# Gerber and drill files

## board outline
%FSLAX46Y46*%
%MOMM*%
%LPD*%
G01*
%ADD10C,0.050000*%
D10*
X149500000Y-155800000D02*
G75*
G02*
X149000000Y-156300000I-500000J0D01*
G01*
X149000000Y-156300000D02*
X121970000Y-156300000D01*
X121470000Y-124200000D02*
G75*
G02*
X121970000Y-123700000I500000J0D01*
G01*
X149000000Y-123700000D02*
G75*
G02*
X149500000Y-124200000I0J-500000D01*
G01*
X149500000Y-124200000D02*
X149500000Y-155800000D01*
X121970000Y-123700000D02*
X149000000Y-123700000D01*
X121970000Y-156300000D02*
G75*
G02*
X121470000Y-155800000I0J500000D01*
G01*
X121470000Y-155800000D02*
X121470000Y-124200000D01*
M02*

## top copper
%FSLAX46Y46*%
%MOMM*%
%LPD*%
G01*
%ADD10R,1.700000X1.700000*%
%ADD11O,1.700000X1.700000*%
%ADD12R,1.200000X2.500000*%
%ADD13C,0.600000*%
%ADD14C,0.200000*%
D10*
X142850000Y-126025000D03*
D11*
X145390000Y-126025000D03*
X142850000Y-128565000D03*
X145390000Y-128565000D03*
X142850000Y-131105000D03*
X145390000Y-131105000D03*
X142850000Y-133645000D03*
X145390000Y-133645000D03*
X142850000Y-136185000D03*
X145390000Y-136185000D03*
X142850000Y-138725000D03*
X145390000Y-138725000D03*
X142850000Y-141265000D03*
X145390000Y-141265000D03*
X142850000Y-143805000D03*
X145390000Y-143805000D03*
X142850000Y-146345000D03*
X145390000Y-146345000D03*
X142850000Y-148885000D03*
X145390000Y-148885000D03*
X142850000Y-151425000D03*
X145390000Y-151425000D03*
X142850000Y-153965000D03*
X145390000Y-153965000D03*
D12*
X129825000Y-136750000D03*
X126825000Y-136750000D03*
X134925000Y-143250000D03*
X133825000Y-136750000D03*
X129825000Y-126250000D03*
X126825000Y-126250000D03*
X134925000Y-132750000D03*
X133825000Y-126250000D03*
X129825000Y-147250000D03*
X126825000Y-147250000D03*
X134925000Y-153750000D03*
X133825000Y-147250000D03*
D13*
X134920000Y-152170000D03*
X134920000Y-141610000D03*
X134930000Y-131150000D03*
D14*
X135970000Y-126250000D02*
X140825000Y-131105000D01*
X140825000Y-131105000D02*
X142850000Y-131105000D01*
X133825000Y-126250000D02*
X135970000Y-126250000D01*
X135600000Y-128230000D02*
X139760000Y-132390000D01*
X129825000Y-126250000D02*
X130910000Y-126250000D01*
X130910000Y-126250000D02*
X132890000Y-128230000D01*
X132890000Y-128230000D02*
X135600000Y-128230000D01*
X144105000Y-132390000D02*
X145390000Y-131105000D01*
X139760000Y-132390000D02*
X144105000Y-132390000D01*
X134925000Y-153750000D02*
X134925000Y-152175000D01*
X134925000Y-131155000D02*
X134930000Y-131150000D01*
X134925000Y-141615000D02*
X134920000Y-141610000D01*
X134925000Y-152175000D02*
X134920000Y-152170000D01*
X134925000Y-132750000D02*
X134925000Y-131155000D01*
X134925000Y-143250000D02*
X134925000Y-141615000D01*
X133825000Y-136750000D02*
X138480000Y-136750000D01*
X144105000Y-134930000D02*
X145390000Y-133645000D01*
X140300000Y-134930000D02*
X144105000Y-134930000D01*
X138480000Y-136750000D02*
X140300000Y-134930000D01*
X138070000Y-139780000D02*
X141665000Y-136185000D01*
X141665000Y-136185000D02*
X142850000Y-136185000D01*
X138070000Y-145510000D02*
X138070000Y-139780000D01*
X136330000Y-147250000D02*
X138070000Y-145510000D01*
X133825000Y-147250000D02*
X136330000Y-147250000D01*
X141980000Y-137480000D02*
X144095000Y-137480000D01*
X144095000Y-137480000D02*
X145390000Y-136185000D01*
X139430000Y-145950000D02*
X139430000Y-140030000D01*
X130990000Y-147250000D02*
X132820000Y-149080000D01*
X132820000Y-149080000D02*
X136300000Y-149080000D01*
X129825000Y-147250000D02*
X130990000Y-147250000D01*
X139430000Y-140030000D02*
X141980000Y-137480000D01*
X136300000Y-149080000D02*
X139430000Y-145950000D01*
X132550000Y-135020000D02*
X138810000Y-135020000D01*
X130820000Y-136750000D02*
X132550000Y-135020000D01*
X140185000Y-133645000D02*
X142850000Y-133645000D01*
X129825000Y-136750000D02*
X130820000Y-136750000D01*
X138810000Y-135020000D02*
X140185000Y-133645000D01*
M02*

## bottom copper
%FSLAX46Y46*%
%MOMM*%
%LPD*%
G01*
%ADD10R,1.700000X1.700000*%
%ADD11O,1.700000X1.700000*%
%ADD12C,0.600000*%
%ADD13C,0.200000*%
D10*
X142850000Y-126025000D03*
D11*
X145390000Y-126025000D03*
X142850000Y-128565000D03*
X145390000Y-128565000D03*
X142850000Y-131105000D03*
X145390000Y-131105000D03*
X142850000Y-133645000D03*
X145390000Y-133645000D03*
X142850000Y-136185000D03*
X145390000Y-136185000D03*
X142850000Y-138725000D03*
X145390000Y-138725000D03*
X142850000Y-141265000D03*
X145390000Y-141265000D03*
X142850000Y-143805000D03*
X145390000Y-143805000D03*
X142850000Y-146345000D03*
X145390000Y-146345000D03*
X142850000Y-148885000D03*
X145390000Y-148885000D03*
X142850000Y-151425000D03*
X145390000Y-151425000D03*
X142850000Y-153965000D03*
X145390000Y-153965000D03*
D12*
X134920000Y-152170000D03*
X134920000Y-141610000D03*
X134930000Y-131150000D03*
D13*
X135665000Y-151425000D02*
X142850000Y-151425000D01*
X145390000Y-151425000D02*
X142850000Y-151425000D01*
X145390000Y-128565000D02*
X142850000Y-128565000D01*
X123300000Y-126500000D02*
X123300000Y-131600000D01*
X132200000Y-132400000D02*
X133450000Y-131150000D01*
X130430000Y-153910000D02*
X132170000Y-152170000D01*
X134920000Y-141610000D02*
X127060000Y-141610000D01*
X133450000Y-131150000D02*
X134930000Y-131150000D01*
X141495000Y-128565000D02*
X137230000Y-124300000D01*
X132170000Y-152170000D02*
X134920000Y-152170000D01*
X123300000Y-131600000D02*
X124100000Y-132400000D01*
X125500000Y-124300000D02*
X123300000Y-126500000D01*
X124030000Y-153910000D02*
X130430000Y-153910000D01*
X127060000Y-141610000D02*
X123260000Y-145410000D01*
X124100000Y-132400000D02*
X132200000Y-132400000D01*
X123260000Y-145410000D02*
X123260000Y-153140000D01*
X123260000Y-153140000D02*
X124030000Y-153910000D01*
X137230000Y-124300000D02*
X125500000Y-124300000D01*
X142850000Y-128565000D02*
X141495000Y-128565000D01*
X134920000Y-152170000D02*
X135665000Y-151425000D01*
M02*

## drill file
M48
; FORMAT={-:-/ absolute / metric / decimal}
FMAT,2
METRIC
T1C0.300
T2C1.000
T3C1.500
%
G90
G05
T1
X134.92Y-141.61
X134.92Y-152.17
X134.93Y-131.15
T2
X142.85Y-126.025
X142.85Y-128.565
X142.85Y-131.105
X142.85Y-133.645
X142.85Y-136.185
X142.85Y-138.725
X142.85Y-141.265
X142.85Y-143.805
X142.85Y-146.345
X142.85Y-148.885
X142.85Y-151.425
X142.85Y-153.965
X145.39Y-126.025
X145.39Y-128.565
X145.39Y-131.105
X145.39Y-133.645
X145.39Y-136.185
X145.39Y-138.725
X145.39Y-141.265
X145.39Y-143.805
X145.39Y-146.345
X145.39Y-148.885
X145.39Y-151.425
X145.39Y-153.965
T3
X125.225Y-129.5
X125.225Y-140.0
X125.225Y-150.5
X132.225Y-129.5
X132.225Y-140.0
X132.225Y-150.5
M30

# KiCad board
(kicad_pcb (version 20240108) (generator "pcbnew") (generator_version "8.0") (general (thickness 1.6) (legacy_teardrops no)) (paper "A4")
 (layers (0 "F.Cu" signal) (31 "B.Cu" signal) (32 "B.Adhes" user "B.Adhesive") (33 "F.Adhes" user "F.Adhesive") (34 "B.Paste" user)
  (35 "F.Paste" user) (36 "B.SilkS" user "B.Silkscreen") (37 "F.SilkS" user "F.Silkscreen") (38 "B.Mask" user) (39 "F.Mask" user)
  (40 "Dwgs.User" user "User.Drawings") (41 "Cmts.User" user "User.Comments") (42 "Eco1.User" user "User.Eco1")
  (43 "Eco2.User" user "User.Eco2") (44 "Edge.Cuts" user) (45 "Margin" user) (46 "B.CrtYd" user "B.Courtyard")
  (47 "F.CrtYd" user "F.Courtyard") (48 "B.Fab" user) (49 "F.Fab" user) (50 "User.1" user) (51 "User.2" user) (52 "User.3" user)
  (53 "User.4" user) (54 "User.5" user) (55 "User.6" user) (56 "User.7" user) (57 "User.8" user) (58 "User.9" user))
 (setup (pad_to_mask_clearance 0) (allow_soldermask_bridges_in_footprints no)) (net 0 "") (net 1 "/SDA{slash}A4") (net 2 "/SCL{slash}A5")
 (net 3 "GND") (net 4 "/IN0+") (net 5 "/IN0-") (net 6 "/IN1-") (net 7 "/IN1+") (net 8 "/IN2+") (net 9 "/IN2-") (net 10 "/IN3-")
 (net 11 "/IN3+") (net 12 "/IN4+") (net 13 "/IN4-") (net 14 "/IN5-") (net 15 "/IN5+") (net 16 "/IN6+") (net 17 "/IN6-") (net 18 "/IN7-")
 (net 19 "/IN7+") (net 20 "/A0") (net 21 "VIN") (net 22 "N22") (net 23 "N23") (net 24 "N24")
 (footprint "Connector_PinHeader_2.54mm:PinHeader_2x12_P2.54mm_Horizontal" (layer "F.Cu") (at 142.85 126.025)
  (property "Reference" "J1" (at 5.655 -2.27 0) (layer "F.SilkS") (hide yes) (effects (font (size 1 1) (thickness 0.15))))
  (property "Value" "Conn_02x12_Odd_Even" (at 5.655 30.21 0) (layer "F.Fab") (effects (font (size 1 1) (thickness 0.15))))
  (pad "1" thru_hole rect (at 0 0) (size 1.7 1.7) (drill 1) (layers "*.Cu" "*.Mask") (remove_unused_layers no) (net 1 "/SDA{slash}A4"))
  (pad "2" thru_hole oval (at 2.54 0) (size 1.7 1.7) (drill 1) (layers "*.Cu" "*.Mask") (remove_unused_layers no) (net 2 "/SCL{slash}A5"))
  (pad "3" thru_hole oval (at 0 2.54) (size 1.7 1.7) (drill 1) (layers "*.Cu" "*.Mask") (remove_unused_layers no) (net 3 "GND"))
  (pad "4" thru_hole oval (at 2.54 2.54) (size 1.7 1.7) (drill 1) (layers "*.Cu" "*.Mask") (remove_unused_layers no) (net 3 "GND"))
  (pad "5" thru_hole oval (at 0 5.08) (size 1.7 1.7) (drill 1) (layers "*.Cu" "*.Mask") (remove_unused_layers no) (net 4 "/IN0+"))
  (pad "6" thru_hole oval (at 2.54 5.08) (size 1.7 1.7) (drill 1) (layers "*.Cu" "*.Mask") (remove_unused_layers no) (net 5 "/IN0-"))
  (pad "7" thru_hole oval (at 0 7.62) (size 1.7 1.7) (drill 1) (layers "*.Cu" "*.Mask") (remove_unused_layers no) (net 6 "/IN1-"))
  (pad "8" thru_hole oval (at 2.54 7.62) (size 1.7 1.7) (drill 1) (layers "*.Cu" "*.Mask") (remove_unused_layers no) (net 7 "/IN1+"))
  (pad "9" thru_hole oval (at 0 10.16) (size 1.7 1.7) (drill 1) (layers "*.Cu" "*.Mask") (remove_unused_layers no) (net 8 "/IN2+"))
  (pad "10" thru_hole oval (at 2.54 10.16) (size 1.7 1.7) (drill 1) (layers "*.Cu" "*.Mask") (remove_unused_layers no) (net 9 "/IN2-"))
  (pad "11" thru_hole oval (at 0 12.7) (size 1.7 1.7) (drill 1) (layers "*.Cu" "*.Mask") (remove_unused_layers no) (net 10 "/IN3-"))
  (pad "12" thru_hole oval (at 2.54 12.7) (size 1.7 1.7) (drill 1) (layers "*.Cu" "*.Mask") (remove_unused_layers no) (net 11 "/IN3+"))
  (pad "13" thru_hole oval (at 0 15.24) (size 1.7 1.7) (drill 1) (layers "*.Cu" "*.Mask") (remove_unused_layers no) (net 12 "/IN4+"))
  (pad "14" thru_hole oval (at 2.54 15.24) (size 1.7 1.7) (drill 1) (layers "*.Cu" "*.Mask") (remove_unused_layers no) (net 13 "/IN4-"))
  (pad "15" thru_hole oval (at 0 17.78) (size 1.7 1.7) (drill 1) (layers "*.Cu" "*.Mask") (remove_unused_layers no) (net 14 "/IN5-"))
  (pad "16" thru_hole oval (at 2.54 17.78) (size 1.7 1.7) (drill 1) (layers "*.Cu" "*.Mask") (remove_unused_layers no) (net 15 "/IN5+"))
  (pad "17" thru_hole oval (at 0 20.32) (size 1.7 1.7) (drill 1) (layers "*.Cu" "*.Mask") (remove_unused_layers no) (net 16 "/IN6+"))
  (pad "18" thru_hole oval (at 2.54 20.32) (size 1.7 1.7) (drill 1) (layers "*.Cu" "*.Mask") (remove_unused_layers no) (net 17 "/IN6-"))
  (pad "19" thru_hole oval (at 0 22.86) (size 1.7 1.7) (drill 1) (layers "*.Cu" "*.Mask") (remove_unused_layers no) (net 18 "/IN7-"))
  (pad "20" thru_hole oval (at 2.54 22.86) (size 1.7 1.7) (drill 1) (layers "*.Cu" "*.Mask") (remove_unused_layers no) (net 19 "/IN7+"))
  (pad "21" thru_hole oval (at 0 25.4) (size 1.7 1.7) (drill 1) (layers "*.Cu" "*.Mask") (remove_unused_layers no) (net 3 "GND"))
  (pad "22" thru_hole oval (at 2.54 25.4) (size 1.7 1.7) (drill 1) (layers "*.Cu" "*.Mask") (remove_unused_layers no) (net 3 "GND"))
  (pad "23" thru_hole oval (at 0 27.94) (size 1.7 1.7) (drill 1) (layers "*.Cu" "*.Mask") (remove_unused_layers no) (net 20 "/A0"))
  (pad "24" thru_hole oval (at 2.54 27.94) (size 1.7 1.7) (drill 1) (layers "*.Cu" "*.Mask") (remove_unused_layers no) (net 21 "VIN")))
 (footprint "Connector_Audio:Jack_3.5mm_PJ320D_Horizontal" (layer "F.Cu") (at 130 140)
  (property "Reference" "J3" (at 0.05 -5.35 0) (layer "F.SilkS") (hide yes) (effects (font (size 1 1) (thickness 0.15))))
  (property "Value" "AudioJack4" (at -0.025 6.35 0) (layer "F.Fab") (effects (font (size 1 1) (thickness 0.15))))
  (pad "" np_thru_hole circle (at -4.775 0) (size 1.5 1.5) (drill 1.5) (layers "*.Cu" "*.Mask"))
  (pad "" np_thru_hole circle (at 2.225 0) (size 1.5 1.5) (drill 1.5) (layers "*.Cu" "*.Mask"))
  (pad "R1" smd rect (at -0.175 -3.25) (size 1.2 2.5) (layers "F.Cu" "F.Paste" "F.Mask") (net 6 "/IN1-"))
  (pad "R2" smd rect (at -3.175 -3.25) (size 1.2 2.5) (layers "F.Cu" "F.Paste" "F.Mask") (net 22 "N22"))
  (pad "S" smd rect (at 4.925 3.25) (size 1.2 2.5) (layers "F.Cu" "F.Paste" "F.Mask") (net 3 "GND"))
  (pad "T" smd rect (at 3.825 -3.25) (size 1.2 2.5) (layers "F.Cu" "F.Paste" "F.Mask") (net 7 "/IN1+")))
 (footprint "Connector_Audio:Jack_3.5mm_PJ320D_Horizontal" (layer "F.Cu") (at 130 129.5)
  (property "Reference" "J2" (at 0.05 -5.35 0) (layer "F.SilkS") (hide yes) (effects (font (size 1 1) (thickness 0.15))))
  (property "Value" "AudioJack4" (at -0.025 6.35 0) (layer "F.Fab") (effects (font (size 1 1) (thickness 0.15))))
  (pad "" np_thru_hole circle (at -4.775 0) (size 1.5 1.5) (drill 1.5) (layers "*.Cu" "*.Mask"))
  (pad "" np_thru_hole circle (at 2.225 0) (size 1.5 1.5) (drill 1.5) (layers "*.Cu" "*.Mask"))
  (pad "R1" smd rect (at -0.175 -3.25) (size 1.2 2.5) (layers "F.Cu" "F.Paste" "F.Mask") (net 5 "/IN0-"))
  (pad "R2" smd rect (at -3.175 -3.25) (size 1.2 2.5) (layers "F.Cu" "F.Paste" "F.Mask") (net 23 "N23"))
  (pad "S" smd rect (at 4.925 3.25) (size 1.2 2.5) (layers "F.Cu" "F.Paste" "F.Mask") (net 3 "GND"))
  (pad "T" smd rect (at 3.825 -3.25) (size 1.2 2.5) (layers "F.Cu" "F.Paste" "F.Mask") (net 4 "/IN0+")))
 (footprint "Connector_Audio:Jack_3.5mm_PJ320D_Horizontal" (layer "F.Cu") (at 130 150.5)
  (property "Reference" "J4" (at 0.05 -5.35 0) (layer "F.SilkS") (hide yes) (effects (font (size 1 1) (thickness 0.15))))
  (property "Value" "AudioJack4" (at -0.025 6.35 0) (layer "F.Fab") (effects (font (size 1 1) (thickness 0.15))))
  (pad "" np_thru_hole circle (at -4.775 0) (size 1.5 1.5) (drill 1.5) (layers "*.Cu" "*.Mask"))
  (pad "" np_thru_hole circle (at 2.225 0) (size 1.5 1.5) (drill 1.5) (layers "*.Cu" "*.Mask"))
  (pad "R1" smd rect (at -0.175 -3.25) (size 1.2 2.5) (layers "F.Cu" "F.Paste" "F.Mask") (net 9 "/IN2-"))
  (pad "R2" smd rect (at -3.175 -3.25) (size 1.2 2.5) (layers "F.Cu" "F.Paste" "F.Mask") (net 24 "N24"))
  (pad "S" smd rect (at 4.925 3.25) (size 1.2 2.5) (layers "F.Cu" "F.Paste" "F.Mask") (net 3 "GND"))
  (pad "T" smd rect (at 3.825 -3.25) (size 1.2 2.5) (layers "F.Cu" "F.Paste" "F.Mask") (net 8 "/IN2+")))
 (gr_arc (start 149.5 155.8) (mid 149.353553 156.153553) (end 149 156.3) (stroke (width 0.05) (type default)) (layer "Edge.Cuts"))
 (gr_line (start 149 156.3) (end 121.97 156.3) (stroke (width 0.05) (type default)) (layer "Edge.Cuts"))
 (gr_arc (start 121.47 124.2) (mid 121.616447 123.846447) (end 121.97 123.7) (stroke (width 0.05) (type default)) (layer "Edge.Cuts"))
 (gr_arc (start 149 123.7) (mid 149.353553 123.846447) (end 149.5 124.2) (stroke (width 0.05) (type default)) (layer "Edge.Cuts"))
 (gr_line (start 149.5 124.2) (end 149.5 155.8) (stroke (width 0.05) (type default)) (layer "Edge.Cuts"))
 (gr_line (start 121.97 123.7) (end 149 123.7) (stroke (width 0.05) (type default)) (layer "Edge.Cuts"))
 (gr_arc (start 121.97 156.3) (mid 121.616447 156.153553) (end 121.47 155.8) (stroke (width 0.05) (type default)) (layer "Edge.Cuts"))
 (gr_line (start 121.47 155.8) (end 121.47 124.2) (stroke (width 0.05) (type default)) (layer "Edge.Cuts"))
 (segment (start 135.97 126.25) (end 140.825 131.105) (width 0.2) (layer "F.Cu") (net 4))
 (segment (start 140.825 131.105) (end 142.85 131.105) (width 0.2) (layer "F.Cu") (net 4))
 (segment (start 133.825 126.25) (end 135.97 126.25) (width 0.2) (layer "F.Cu") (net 4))
 (segment (start 135.6 128.23) (end 139.76 132.39) (width 0.2) (layer "F.Cu") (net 5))
 (segment (start 129.825 126.25) (end 130.91 126.25) (width 0.2) (layer "F.Cu") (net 5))
 (segment (start 130.91 126.25) (end 132.89 128.23) (width 0.2) (layer "F.Cu") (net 5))
 (segment (start 132.89 128.23) (end 135.6 128.23) (width 0.2) (layer "F.Cu") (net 5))
 (segment (start 144.105 132.39) (end 145.39 131.105) (width 0.2) (layer "F.Cu") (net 5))
 (segment (start 139.76 132.39) (end 144.105 132.39) (width 0.2) (layer "F.Cu") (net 5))
 (segment (start 134.925 153.75) (end 134.925 152.175) (width 0.2) (layer "F.Cu") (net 3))
 (segment (start 134.925 131.155) (end 134.93 131.15) (width 0.2) (layer "F.Cu") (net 3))
 (segment (start 134.925 141.615) (end 134.92 141.61) (width 0.2) (layer "F.Cu") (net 3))
 (segment (start 134.925 152.175) (end 134.92 152.17) (width 0.2) (layer "F.Cu") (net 3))
 (segment (start 134.925 132.75) (end 134.925 131.155) (width 0.2) (layer "F.Cu") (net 3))
 (segment (start 134.925 143.25) (end 134.925 141.615) (width 0.2) (layer "F.Cu") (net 3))
 (via (at 134.92 152.17) (size 0.6) (drill 0.3) (layers "F.Cu" "B.Cu") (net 3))
 (via (at 134.92 141.61) (size 0.6) (drill 0.3) (layers "F.Cu" "B.Cu") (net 3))
 (via (at 134.93 131.15) (size 0.6) (drill 0.3) (layers "F.Cu" "B.Cu") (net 3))
 (segment (start 135.665 151.425) (end 142.85 151.425) (width 0.2) (layer "B.Cu") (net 3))
 (segment (start 145.39 151.425) (end 142.85 151.425) (width 0.2) (layer "B.Cu") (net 3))
 (segment (start 145.39 128.565) (end 142.85 128.565) (width 0.2) (layer "B.Cu") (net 3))
 (segment (start 123.3 126.5) (end 123.3 131.6) (width 0.2) (layer "B.Cu") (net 3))
 (segment (start 132.2 132.4) (end 133.45 131.15) (width 0.2) (layer "B.Cu") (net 3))
 (segment (start 130.43 153.91) (end 132.17 152.17) (width 0.2) (layer "B.Cu") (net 3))
 (segment (start 134.92 141.61) (end 127.06 141.61) (width 0.2) (layer "B.Cu") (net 3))
 (segment (start 133.45 131.15) (end 134.93 131.15) (width 0.2) (layer "B.Cu") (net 3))
 (segment (start 141.495 128.565) (end 137.23 124.3) (width 0.2) (layer "B.Cu") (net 3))
 (segment (start 132.17 152.17) (end 134.92 152.17) (width 0.2) (layer "B.Cu") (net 3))
 (segment (start 123.3 131.6) (end 124.1 132.4) (width 0.2) (layer "B.Cu") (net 3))
 (segment (start 125.5 124.3) (end 123.3 126.5) (width 0.2) (layer "B.Cu") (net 3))
 (segment (start 124.03 153.91) (end 130.43 153.91) (width 0.2) (layer "B.Cu") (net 3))
 (segment (start 127.06 141.61) (end 123.26 145.41) (width 0.2) (layer "B.Cu") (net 3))
 (segment (start 124.1 132.4) (end 132.2 132.4) (width 0.2) (layer "B.Cu") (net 3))
 (segment (start 123.26 145.41) (end 123.26 153.14) (width 0.2) (layer "B.Cu") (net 3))
 (segment (start 123.26 153.14) (end 124.03 153.91) (width 0.2) (layer "B.Cu") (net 3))
 (segment (start 137.23 124.3) (end 125.5 124.3) (width 0.2) (layer "B.Cu") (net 3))
 (segment (start 142.85 128.565) (end 141.495 128.565) (width 0.2) (layer "B.Cu") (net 3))
 (segment (start 134.92 152.17) (end 135.665 151.425) (width 0.2) (layer "B.Cu") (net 3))
 (segment (start 133.825 136.75) (end 138.48 136.75) (width 0.2) (layer "F.Cu") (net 7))
 (segment (start 144.105 134.93) (end 145.39 133.645) (width 0.2) (layer "F.Cu") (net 7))
 (segment (start 140.3 134.93) (end 144.105 134.93) (width 0.2) (layer "F.Cu") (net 7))
 (segment (start 138.48 136.75) (end 140.3 134.93) (width 0.2) (layer "F.Cu") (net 7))
 (segment (start 138.07 139.78) (end 141.665 136.185) (width 0.2) (layer "F.Cu") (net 8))
 (segment (start 141.665 136.185) (end 142.85 136.185) (width 0.2) (layer "F.Cu") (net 8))
 (segment (start 138.07 145.51) (end 138.07 139.78) (width 0.2) (layer "F.Cu") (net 8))
 (segment (start 136.33 147.25) (end 138.07 145.51) (width 0.2) (layer "F.Cu") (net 8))
 (segment (start 133.825 147.25) (end 136.33 147.25) (width 0.2) (layer "F.Cu") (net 8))
 (segment (start 141.98 137.48) (end 144.095 137.48) (width 0.2) (layer "F.Cu") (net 9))
 (segment (start 144.095 137.48) (end 145.39 136.185) (width 0.2) (layer "F.Cu") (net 9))
 (segment (start 139.43 145.95) (end 139.43 140.03) (width 0.2) (layer "F.Cu") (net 9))
 (segment (start 130.99 147.25) (end 132.82 149.08) (width 0.2) (layer "F.Cu") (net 9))
 (segment (start 132.82 149.08) (end 136.3 149.08) (width 0.2) (layer "F.Cu") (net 9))
 (segment (start 129.825 147.25) (end 130.99 147.25) (width 0.2) (layer "F.Cu") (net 9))
 (segment (start 139.43 140.03) (end 141.98 137.48) (width 0.2) (layer "F.Cu") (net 9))
 (segment (start 136.3 149.08) (end 139.43 145.95) (width 0.2) (layer "F.Cu") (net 9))
 (segment (start 132.55 135.02) (end 138.81 135.02) (width 0.2) (layer "F.Cu") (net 6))
 (segment (start 130.82 136.75) (end 132.55 135.02) (width 0.2) (layer "F.Cu") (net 6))
 (segment (start 140.185 133.645) (end 142.85 133.645) (width 0.2) (layer "F.Cu") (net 6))
 (segment (start 129.825 136.75) (end 130.82 136.75) (width 0.2) (layer "F.Cu") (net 6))
 (segment (start 138.81 135.02) (end 140.185 133.645) (width 0.2) (layer "F.Cu") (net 6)))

